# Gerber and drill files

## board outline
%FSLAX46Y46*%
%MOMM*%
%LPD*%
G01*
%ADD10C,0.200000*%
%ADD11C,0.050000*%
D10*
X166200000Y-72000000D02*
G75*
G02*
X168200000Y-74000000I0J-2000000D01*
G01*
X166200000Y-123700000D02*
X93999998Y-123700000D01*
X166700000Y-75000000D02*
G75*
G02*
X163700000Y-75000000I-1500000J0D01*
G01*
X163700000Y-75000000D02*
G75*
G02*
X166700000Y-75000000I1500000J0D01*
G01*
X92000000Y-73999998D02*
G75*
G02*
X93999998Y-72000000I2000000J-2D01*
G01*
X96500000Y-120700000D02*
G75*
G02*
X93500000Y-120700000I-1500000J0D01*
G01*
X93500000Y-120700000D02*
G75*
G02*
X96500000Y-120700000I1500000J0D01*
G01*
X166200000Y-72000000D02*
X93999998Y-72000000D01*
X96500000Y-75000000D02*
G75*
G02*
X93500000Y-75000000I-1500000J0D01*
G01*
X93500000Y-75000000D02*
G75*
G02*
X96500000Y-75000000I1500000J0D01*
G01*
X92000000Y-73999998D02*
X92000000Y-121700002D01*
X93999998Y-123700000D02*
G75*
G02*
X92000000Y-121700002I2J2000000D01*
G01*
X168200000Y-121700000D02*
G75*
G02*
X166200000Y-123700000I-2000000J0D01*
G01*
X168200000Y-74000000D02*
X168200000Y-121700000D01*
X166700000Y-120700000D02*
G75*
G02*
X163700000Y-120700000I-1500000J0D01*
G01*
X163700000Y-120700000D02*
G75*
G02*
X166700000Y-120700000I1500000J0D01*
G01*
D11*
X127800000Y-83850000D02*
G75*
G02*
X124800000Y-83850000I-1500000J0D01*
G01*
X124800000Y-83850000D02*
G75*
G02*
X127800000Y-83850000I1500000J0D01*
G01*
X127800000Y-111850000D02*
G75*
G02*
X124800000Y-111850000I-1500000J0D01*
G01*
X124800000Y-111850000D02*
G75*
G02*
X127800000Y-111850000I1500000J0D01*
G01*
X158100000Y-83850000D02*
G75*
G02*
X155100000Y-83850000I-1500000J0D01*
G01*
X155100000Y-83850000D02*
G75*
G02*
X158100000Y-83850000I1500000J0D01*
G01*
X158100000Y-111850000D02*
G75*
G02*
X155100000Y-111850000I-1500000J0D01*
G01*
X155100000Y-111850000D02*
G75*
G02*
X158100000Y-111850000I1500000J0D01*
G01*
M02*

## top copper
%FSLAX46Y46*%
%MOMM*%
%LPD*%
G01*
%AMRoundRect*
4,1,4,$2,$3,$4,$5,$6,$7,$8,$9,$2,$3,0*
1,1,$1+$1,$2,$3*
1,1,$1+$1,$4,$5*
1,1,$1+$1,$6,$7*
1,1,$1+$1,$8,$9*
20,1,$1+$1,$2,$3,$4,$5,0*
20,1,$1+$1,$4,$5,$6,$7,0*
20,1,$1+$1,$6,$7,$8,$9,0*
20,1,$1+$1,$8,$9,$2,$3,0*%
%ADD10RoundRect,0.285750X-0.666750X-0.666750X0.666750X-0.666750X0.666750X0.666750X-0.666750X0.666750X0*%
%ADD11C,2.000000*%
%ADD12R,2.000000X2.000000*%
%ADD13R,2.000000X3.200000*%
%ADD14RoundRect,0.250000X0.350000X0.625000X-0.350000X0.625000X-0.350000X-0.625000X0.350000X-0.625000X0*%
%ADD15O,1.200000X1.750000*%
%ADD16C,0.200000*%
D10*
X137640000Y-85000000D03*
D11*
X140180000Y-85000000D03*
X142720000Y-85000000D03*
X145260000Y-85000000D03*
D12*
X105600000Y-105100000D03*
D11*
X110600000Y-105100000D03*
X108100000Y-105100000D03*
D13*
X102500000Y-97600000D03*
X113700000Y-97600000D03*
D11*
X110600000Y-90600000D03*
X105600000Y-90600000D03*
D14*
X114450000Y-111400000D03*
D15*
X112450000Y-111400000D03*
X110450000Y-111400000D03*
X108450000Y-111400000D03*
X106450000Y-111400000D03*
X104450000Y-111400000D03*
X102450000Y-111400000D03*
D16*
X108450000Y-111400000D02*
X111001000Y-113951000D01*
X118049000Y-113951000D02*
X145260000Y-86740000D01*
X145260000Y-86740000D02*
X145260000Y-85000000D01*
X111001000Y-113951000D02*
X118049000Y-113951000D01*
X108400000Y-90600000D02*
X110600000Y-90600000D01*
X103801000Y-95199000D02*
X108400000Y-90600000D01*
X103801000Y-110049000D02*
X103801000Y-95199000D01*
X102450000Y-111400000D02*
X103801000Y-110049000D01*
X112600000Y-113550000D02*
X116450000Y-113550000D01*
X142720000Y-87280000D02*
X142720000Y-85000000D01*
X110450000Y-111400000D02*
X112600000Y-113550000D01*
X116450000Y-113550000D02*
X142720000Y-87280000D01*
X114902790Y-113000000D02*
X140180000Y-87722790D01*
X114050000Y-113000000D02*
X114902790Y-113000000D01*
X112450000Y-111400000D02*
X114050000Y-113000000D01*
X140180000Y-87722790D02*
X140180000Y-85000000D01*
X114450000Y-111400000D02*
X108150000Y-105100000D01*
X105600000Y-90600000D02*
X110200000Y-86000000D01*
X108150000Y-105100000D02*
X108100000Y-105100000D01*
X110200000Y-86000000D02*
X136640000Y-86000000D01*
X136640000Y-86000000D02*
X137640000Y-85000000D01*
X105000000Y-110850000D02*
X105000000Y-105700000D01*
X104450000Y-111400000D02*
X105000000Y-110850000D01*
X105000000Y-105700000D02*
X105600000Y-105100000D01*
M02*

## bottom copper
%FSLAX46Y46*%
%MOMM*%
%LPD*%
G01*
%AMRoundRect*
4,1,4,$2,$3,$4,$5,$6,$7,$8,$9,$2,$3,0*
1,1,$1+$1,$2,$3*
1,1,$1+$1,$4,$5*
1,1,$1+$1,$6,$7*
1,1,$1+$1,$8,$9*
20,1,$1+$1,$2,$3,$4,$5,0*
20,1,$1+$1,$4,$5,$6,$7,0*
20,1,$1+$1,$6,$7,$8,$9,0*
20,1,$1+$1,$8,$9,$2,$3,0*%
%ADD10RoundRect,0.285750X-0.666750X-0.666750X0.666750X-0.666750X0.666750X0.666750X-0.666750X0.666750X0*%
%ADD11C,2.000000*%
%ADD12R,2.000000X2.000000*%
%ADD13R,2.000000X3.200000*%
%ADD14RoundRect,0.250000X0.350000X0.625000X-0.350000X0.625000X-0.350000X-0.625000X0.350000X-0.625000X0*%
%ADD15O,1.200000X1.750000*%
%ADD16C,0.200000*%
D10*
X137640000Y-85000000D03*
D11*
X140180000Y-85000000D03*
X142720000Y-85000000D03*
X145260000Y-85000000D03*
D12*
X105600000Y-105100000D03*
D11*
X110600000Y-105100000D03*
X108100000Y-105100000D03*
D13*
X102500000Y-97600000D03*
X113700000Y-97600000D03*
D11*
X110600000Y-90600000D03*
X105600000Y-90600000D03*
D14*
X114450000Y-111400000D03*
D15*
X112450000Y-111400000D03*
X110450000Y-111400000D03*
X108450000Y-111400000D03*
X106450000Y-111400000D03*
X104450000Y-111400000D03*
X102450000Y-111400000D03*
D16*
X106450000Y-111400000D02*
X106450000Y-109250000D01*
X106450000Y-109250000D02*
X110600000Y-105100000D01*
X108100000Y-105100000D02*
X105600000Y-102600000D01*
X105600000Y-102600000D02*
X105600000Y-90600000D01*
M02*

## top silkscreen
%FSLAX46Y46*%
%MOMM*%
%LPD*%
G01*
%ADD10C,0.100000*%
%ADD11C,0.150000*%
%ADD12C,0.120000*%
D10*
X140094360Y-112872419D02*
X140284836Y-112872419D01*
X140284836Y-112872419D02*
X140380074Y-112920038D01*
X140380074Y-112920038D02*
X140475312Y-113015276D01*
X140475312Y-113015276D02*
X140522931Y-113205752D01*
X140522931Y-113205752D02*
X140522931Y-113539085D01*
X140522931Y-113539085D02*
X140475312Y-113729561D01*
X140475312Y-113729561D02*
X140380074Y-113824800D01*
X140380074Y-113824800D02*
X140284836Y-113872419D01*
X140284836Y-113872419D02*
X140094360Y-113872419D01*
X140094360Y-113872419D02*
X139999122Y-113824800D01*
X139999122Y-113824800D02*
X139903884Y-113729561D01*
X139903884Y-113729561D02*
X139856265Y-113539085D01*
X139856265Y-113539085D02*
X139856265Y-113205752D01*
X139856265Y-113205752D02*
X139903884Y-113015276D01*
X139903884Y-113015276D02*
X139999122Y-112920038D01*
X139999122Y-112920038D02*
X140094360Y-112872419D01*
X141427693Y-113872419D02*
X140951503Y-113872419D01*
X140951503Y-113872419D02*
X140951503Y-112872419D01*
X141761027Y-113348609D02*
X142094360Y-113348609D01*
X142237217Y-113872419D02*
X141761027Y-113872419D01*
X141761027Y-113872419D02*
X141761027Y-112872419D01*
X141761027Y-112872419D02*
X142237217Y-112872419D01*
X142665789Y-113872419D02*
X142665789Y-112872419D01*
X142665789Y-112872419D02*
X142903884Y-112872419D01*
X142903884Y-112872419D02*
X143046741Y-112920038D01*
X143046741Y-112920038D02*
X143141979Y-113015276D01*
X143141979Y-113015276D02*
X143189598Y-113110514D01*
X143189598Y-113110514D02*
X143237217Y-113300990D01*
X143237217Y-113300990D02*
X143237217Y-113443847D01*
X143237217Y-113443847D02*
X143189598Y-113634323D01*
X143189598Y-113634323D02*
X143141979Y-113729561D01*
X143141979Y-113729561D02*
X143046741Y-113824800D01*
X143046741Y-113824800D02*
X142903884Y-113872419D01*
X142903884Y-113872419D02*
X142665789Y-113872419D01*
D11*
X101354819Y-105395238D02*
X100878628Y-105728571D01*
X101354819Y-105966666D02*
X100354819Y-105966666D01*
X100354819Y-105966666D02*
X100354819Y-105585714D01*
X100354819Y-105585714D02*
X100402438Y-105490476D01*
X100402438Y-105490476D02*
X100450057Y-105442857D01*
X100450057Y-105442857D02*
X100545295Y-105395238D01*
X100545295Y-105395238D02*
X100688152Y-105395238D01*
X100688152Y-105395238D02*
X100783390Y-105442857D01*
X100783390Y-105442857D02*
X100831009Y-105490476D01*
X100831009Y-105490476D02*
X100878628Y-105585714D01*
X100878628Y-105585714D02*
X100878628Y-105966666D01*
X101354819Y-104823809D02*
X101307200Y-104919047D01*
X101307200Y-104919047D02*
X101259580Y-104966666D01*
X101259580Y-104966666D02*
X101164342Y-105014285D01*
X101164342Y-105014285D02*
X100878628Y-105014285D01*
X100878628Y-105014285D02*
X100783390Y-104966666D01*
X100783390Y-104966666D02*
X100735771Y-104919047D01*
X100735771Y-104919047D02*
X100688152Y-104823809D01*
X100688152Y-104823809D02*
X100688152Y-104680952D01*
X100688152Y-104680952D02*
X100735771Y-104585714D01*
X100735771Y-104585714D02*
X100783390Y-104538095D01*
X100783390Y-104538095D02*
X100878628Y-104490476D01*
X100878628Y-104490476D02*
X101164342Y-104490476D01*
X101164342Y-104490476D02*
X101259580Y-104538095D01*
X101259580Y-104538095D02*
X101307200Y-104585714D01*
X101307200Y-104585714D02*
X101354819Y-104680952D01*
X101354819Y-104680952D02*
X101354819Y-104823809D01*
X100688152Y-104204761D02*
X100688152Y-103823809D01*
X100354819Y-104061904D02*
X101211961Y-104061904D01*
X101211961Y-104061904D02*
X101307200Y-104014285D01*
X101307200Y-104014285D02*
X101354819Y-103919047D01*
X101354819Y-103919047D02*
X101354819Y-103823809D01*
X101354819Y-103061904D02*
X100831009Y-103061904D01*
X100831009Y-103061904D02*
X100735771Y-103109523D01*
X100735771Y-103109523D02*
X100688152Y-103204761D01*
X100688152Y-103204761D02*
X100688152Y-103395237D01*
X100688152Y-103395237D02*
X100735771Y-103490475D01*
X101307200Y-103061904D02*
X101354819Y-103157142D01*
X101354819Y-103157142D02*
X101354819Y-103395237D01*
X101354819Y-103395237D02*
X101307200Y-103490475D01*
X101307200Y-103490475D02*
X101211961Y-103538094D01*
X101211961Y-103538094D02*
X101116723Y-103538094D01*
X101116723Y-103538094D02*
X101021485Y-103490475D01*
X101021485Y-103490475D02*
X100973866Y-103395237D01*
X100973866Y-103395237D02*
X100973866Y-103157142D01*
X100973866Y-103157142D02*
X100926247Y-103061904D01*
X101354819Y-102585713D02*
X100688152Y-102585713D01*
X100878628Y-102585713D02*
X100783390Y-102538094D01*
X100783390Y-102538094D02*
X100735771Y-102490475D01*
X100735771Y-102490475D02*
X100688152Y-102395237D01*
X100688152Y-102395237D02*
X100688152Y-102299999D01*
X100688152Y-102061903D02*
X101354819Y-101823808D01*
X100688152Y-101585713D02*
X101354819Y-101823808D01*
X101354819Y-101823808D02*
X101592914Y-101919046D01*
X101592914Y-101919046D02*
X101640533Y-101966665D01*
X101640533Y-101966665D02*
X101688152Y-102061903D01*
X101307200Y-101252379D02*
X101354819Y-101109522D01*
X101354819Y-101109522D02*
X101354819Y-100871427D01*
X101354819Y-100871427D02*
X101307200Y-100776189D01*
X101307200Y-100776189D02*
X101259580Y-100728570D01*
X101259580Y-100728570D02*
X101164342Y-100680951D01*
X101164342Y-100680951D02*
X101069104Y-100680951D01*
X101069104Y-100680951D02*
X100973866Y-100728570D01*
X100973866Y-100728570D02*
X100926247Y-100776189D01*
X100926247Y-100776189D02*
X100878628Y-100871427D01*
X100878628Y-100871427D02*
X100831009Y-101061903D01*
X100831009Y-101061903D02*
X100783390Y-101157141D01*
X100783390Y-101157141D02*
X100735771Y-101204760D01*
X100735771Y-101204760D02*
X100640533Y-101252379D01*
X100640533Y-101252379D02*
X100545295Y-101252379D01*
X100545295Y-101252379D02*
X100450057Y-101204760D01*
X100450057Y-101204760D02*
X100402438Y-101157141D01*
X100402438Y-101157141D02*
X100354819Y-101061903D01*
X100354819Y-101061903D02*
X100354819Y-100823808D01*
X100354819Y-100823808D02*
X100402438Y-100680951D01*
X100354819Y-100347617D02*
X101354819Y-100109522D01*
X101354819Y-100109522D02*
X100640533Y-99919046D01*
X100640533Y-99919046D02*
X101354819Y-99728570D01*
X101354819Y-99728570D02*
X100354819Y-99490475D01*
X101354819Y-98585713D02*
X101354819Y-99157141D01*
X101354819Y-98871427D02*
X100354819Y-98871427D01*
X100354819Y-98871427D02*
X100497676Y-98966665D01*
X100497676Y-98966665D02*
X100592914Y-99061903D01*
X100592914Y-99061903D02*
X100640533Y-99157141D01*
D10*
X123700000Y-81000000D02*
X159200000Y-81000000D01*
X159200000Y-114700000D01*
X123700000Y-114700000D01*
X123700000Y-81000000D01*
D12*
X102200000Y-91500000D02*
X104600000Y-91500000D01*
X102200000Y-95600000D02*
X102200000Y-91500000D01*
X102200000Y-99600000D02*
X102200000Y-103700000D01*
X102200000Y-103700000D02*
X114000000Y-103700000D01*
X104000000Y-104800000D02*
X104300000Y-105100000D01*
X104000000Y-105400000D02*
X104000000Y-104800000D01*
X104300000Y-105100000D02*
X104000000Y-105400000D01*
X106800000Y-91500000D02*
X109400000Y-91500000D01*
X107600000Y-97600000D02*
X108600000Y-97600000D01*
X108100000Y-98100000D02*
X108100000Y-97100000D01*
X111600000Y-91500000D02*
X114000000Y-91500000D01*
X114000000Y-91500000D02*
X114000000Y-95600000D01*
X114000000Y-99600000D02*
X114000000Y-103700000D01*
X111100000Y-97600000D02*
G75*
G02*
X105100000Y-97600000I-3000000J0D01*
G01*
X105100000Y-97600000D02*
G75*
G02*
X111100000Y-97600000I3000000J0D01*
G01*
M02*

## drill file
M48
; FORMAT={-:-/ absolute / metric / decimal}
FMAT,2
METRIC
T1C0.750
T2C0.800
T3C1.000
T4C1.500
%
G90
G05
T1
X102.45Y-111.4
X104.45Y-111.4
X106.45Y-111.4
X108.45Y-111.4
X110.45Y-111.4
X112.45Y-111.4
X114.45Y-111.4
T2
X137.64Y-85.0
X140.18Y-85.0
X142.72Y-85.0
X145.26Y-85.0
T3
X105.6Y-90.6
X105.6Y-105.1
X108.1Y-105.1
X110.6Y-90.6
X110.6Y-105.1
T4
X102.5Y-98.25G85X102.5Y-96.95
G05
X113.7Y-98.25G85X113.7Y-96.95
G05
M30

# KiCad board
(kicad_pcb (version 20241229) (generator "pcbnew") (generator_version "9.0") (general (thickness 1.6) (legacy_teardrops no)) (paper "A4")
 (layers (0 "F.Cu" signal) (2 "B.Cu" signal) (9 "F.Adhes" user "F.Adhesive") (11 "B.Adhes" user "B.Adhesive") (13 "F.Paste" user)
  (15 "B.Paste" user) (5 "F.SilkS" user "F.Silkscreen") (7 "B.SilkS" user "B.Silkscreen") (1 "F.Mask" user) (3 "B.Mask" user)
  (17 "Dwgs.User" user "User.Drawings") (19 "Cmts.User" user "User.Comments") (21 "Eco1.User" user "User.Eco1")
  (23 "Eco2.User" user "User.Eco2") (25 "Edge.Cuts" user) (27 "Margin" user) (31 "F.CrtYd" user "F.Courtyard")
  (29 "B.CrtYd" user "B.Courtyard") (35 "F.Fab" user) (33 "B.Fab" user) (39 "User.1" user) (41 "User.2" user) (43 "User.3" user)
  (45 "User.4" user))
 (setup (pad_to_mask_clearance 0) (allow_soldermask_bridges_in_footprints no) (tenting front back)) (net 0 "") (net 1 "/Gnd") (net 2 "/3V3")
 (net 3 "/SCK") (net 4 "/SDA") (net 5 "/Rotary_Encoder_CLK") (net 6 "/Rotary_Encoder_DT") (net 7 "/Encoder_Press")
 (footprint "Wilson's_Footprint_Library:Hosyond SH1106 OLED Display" (layer "F.Cu") (at 123.7 114.7)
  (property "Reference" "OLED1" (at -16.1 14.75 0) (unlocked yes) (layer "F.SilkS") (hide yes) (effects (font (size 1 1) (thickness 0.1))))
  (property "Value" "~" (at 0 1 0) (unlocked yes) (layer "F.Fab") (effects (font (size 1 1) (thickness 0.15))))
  (fp_rect (start 0 -33.7) (end 35.5 0) (stroke (width 0.1) (type default)) (fill no) (layer "F.SilkS"))
  (fp_circle (center 2.6 -30.85) (end 4.1 -30.85) (stroke (width 0.05) (type default)) (fill no) (layer "Edge.Cuts"))
  (fp_circle (center 2.6 -2.85) (end 4.1 -2.85) (stroke (width 0.05) (type default)) (fill no) (layer "Edge.Cuts"))
  (fp_circle (center 32.9 -30.85) (end 34.4 -30.85) (stroke (width 0.05) (type default)) (fill no) (layer "Edge.Cuts"))
  (fp_circle (center 32.9 -2.85) (end 34.4 -2.85) (stroke (width 0.05) (type default)) (fill no) (layer "Edge.Cuts"))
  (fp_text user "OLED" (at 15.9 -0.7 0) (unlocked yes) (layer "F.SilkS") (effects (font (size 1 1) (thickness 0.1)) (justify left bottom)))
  (pad "1" thru_hole roundrect (at 13.94 -29.7) (size 1.905 1.905) (drill 0.8) (layers "*.Cu" "*.Mask") (remove_unused_layers no)
   (roundrect_rratio 0.15) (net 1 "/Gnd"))
  (pad "2" thru_hole circle (at 16.48 -29.7) (size 2 2) (drill 0.8) (layers "*.Cu" "*.Mask") (remove_unused_layers no) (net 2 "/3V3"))
  (pad "3" thru_hole circle (at 19.02 -29.7) (size 2 2) (drill 0.8) (layers "*.Cu" "*.Mask") (remove_unused_layers no) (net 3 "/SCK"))
  (pad "4" thru_hole circle (at 21.56 -29.7) (size 2 2) (drill 0.8) (layers "*.Cu" "*.Mask") (remove_unused_layers no) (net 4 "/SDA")))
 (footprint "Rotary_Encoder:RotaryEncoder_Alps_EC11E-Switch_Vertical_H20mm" (layer "F.Cu") (at 105.6 105.1 90)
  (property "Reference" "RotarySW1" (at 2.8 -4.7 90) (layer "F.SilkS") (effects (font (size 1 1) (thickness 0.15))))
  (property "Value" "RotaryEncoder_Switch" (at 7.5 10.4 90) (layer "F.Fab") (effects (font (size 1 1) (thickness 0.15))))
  (fp_line (start 13.6 -3.4) (end 13.6 -1) (stroke (width 0.12) (type solid)) (layer "F.SilkS"))
  (fp_line (start 9.5 -3.4) (end 13.6 -3.4) (stroke (width 0.12) (type solid)) (layer "F.SilkS"))
  (fp_line (start 5.5 -3.4) (end 1.4 -3.4) (stroke (width 0.12) (type solid)) (layer "F.SilkS"))
  (fp_line (start 1.4 -3.4) (end 1.4 8.4) (stroke (width 0.12) (type solid)) (layer "F.SilkS"))
  (fp_line (start 0.3 -1.6) (end 0 -1.3) (stroke (width 0.12) (type solid)) (layer "F.SilkS"))
  (fp_line (start -0.3 -1.6) (end 0.3 -1.6) (stroke (width 0.12) (type solid)) (layer "F.SilkS"))
  (fp_line (start 0 -1.3) (end -0.3 -1.6) (stroke (width 0.12) (type solid)) (layer "F.SilkS"))
  (fp_line (start 13.6 1.2) (end 13.6 3.8) (stroke (width 0.12) (type solid)) (layer "F.SilkS"))
  (fp_line (start 7.5 2) (end 7.5 3) (stroke (width 0.12) (type solid)) (layer "F.SilkS"))
  (fp_line (start 7 2.5) (end 8 2.5) (stroke (width 0.12) (type solid)) (layer "F.SilkS"))
  (fp_line (start 13.6 6) (end 13.6 8.4) (stroke (width 0.12) (type solid)) (layer "F.SilkS"))
  (fp_line (start 13.6 8.4) (end 9.5 8.4) (stroke (width 0.12) (type solid)) (layer "F.SilkS"))
  (fp_line (start 5.5 8.4) (end 1.4 8.4) (stroke (width 0.12) (type solid)) (layer "F.SilkS"))
  (fp_circle (center 7.5 2.5) (end 10.5 2.5) (stroke (width 0.12) (type solid)) (fill no) (layer "F.SilkS"))
  (pad "A" thru_hole rect (at 0 0 90) (size 2 2) (drill 1) (layers "*.Cu" "*.Mask") (remove_unused_layers no) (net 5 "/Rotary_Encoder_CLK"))
  (pad "B" thru_hole circle (at 0 5 90) (size 2 2) (drill 1) (layers "*.Cu" "*.Mask") (remove_unused_layers no) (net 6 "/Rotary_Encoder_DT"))
  (pad "C" thru_hole circle (at 0 2.5 90) (size 2 2) (drill 1) (layers "*.Cu" "*.Mask") (remove_unused_layers no) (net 1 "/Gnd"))
  (pad "MP" thru_hole rect (at 7.5 -3.1 90) (size 3.2 2) (drill oval 2.8 1.5) (layers "*.Cu" "*.Mask") (remove_unused_layers no))
  (pad "MP" thru_hole rect (at 7.5 8.1 90) (size 3.2 2) (drill oval 2.8 1.5) (layers "*.Cu" "*.Mask") (remove_unused_layers no))
  (pad "S1" thru_hole circle (at 14.5 5 90) (size 2 2) (drill 1) (layers "*.Cu" "*.Mask") (remove_unused_layers no) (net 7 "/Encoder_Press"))
  (pad "S2" thru_hole circle (at 14.5 0 90) (size 2 2) (drill 1) (layers "*.Cu" "*.Mask") (remove_unused_layers no) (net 1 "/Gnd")))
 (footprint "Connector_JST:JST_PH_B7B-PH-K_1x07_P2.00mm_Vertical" (layer "B.Cu") (at 114.45 111.4 180)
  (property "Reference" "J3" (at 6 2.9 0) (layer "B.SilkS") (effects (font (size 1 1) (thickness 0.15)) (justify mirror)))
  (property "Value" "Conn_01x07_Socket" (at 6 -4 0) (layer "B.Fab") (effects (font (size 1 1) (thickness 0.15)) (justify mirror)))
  (pad "1" thru_hole roundrect (at 0 0 180) (size 1.2 1.75) (drill 0.75) (layers "*.Cu" "*.Mask") (remove_unused_layers no)
   (roundrect_rratio 0.208333) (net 1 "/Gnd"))
  (pad "2" thru_hole oval (at 2 0 180) (size 1.2 1.75) (drill 0.75) (layers "*.Cu" "*.Mask") (remove_unused_layers no) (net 2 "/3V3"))
  (pad "3" thru_hole oval (at 4 0 180) (size 1.2 1.75) (drill 0.75) (layers "*.Cu" "*.Mask") (remove_unused_layers no) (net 3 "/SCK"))
  (pad "4" thru_hole oval (at 6 0 180) (size 1.2 1.75) (drill 0.75) (layers "*.Cu" "*.Mask") (remove_unused_layers no) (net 4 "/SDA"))
  (pad "5" thru_hole oval (at 8 0 180) (size 1.2 1.75) (drill 0.75) (layers "*.Cu" "*.Mask") (remove_unused_layers no)
   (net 6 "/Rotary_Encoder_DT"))
  (pad "6" thru_hole oval (at 10 0 180) (size 1.2 1.75) (drill 0.75) (layers "*.Cu" "*.Mask") (remove_unused_layers no)
   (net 5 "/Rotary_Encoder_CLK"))
  (pad "7" thru_hole oval (at 12 0 180) (size 1.2 1.75) (drill 0.75) (layers "*.Cu" "*.Mask") (remove_unused_layers no)
   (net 7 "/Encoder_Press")))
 (gr_arc (start 166.2 72) (mid 167.614214 72.585786) (end 168.2 74) (stroke (width 0.2) (type default)) (layer "Edge.Cuts"))
 (gr_line (start 166.2 123.7) (end 93.999998 123.7) (stroke (width 0.2) (type default)) (layer "Edge.Cuts"))
 (gr_circle (center 165.2 75) (end 166.7 75) (stroke (width 0.2) (type default)) (fill no) (layer "Edge.Cuts"))
 (gr_arc (start 92 73.999998) (mid 92.585786 72.585786) (end 93.999998 72) (stroke (width 0.2) (type default)) (layer "Edge.Cuts"))
 (gr_circle (center 95 120.7) (end 96.5 120.7) (stroke (width 0.2) (type default)) (fill no) (layer "Edge.Cuts"))
 (gr_line (start 166.2 72) (end 93.999998 72) (stroke (width 0.2) (type default)) (layer "Edge.Cuts"))
 (gr_circle (center 95 75) (end 96.5 75) (stroke (width 0.2) (type default)) (fill no) (layer "Edge.Cuts"))
 (gr_line (start 92 73.999998) (end 92 121.700002) (stroke (width 0.2) (type default)) (layer "Edge.Cuts"))
 (gr_arc (start 93.999998 123.7) (mid 92.585786 123.114214) (end 92 121.700002) (stroke (width 0.2) (type default)) (layer "Edge.Cuts"))
 (gr_arc (start 168.2 121.7) (mid 167.614214 123.114214) (end 166.2 123.7) (stroke (width 0.2) (type default)) (layer "Edge.Cuts"))
 (gr_line (start 168.2 74) (end 168.2 121.7) (stroke (width 0.2) (type default)) (layer "Edge.Cuts"))
 (gr_circle (center 165.2 120.7) (end 166.7 120.7) (stroke (width 0.2) (type default)) (fill no) (layer "Edge.Cuts"))
 (segment (start 106.45 111.4) (end 106.45 109.25) (width 0.2) (layer "B.Cu") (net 6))
 (segment (start 106.45 109.25) (end 110.6 105.1) (width 0.2) (layer "B.Cu") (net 6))
 (segment (start 108.45 111.4) (end 111.001 113.951) (width 0.2) (layer "F.Cu") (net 4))
 (segment (start 118.049 113.951) (end 145.26 86.74) (width 0.2) (layer "F.Cu") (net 4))
 (segment (start 145.26 86.74) (end 145.26 85) (width 0.2) (layer "F.Cu") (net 4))
 (segment (start 111.001 113.951) (end 118.049 113.951) (width 0.2) (layer "F.Cu") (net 4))
 (segment (start 108.4 90.6) (end 110.6 90.6) (width 0.2) (layer "F.Cu") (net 7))
 (segment (start 103.801 95.199) (end 108.4 90.6) (width 0.2) (layer "F.Cu") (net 7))
 (segment (start 103.801 110.049) (end 103.801 95.199) (width 0.2) (layer "F.Cu") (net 7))
 (segment (start 102.45 111.4) (end 103.801 110.049) (width 0.2) (layer "F.Cu") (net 7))
 (segment (start 112.6 113.55) (end 116.45 113.55) (width 0.2) (layer "F.Cu") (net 3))
 (segment (start 142.72 87.28) (end 142.72 85) (width 0.2) (layer "F.Cu") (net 3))
 (segment (start 110.45 111.4) (end 112.6 113.55) (width 0.2) (layer "F.Cu") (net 3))
 (segment (start 116.45 113.55) (end 142.72 87.28) (width 0.2) (layer "F.Cu") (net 3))
 (segment (start 114.90279 113) (end 140.18 87.72279) (width 0.2) (layer "F.Cu") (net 2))
 (segment (start 114.05 113) (end 114.90279 113) (width 0.2) (layer "F.Cu") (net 2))
 (segment (start 112.45 111.4) (end 114.05 113) (width 0.2) (layer "F.Cu") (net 2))
 (segment (start 140.18 87.72279) (end 140.18 85) (width 0.2) (layer "F.Cu") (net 2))
 (segment (start 114.45 111.4) (end 108.15 105.1) (width 0.2) (layer "F.Cu") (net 1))
 (segment (start 105.6 90.6) (end 110.2 86) (width 0.2) (layer "F.Cu") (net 1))
 (segment (start 108.15 105.1) (end 108.1 105.1) (width 0.2) (layer "F.Cu") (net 1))
 (segment (start 110.2 86) (end 136.64 86) (width 0.2) (layer "F.Cu") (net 1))
 (segment (start 136.64 86) (end 137.64 85) (width 0.2) (layer "F.Cu") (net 1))
 (segment (start 108.1 105.1) (end 105.6 102.6) (width 0.2) (layer "B.Cu") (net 1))
 (segment (start 105.6 102.6) (end 105.6 90.6) (width 0.2) (layer "B.Cu") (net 1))
 (segment (start 105 110.85) (end 105 105.7) (width 0.2) (layer "F.Cu") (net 5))
 (segment (start 104.45 111.4) (end 105 110.85) (width 0.2) (layer "F.Cu") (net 5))
 (segment (start 105 105.7) (end 105.6 105.1) (width 0.2) (layer "F.Cu") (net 5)))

